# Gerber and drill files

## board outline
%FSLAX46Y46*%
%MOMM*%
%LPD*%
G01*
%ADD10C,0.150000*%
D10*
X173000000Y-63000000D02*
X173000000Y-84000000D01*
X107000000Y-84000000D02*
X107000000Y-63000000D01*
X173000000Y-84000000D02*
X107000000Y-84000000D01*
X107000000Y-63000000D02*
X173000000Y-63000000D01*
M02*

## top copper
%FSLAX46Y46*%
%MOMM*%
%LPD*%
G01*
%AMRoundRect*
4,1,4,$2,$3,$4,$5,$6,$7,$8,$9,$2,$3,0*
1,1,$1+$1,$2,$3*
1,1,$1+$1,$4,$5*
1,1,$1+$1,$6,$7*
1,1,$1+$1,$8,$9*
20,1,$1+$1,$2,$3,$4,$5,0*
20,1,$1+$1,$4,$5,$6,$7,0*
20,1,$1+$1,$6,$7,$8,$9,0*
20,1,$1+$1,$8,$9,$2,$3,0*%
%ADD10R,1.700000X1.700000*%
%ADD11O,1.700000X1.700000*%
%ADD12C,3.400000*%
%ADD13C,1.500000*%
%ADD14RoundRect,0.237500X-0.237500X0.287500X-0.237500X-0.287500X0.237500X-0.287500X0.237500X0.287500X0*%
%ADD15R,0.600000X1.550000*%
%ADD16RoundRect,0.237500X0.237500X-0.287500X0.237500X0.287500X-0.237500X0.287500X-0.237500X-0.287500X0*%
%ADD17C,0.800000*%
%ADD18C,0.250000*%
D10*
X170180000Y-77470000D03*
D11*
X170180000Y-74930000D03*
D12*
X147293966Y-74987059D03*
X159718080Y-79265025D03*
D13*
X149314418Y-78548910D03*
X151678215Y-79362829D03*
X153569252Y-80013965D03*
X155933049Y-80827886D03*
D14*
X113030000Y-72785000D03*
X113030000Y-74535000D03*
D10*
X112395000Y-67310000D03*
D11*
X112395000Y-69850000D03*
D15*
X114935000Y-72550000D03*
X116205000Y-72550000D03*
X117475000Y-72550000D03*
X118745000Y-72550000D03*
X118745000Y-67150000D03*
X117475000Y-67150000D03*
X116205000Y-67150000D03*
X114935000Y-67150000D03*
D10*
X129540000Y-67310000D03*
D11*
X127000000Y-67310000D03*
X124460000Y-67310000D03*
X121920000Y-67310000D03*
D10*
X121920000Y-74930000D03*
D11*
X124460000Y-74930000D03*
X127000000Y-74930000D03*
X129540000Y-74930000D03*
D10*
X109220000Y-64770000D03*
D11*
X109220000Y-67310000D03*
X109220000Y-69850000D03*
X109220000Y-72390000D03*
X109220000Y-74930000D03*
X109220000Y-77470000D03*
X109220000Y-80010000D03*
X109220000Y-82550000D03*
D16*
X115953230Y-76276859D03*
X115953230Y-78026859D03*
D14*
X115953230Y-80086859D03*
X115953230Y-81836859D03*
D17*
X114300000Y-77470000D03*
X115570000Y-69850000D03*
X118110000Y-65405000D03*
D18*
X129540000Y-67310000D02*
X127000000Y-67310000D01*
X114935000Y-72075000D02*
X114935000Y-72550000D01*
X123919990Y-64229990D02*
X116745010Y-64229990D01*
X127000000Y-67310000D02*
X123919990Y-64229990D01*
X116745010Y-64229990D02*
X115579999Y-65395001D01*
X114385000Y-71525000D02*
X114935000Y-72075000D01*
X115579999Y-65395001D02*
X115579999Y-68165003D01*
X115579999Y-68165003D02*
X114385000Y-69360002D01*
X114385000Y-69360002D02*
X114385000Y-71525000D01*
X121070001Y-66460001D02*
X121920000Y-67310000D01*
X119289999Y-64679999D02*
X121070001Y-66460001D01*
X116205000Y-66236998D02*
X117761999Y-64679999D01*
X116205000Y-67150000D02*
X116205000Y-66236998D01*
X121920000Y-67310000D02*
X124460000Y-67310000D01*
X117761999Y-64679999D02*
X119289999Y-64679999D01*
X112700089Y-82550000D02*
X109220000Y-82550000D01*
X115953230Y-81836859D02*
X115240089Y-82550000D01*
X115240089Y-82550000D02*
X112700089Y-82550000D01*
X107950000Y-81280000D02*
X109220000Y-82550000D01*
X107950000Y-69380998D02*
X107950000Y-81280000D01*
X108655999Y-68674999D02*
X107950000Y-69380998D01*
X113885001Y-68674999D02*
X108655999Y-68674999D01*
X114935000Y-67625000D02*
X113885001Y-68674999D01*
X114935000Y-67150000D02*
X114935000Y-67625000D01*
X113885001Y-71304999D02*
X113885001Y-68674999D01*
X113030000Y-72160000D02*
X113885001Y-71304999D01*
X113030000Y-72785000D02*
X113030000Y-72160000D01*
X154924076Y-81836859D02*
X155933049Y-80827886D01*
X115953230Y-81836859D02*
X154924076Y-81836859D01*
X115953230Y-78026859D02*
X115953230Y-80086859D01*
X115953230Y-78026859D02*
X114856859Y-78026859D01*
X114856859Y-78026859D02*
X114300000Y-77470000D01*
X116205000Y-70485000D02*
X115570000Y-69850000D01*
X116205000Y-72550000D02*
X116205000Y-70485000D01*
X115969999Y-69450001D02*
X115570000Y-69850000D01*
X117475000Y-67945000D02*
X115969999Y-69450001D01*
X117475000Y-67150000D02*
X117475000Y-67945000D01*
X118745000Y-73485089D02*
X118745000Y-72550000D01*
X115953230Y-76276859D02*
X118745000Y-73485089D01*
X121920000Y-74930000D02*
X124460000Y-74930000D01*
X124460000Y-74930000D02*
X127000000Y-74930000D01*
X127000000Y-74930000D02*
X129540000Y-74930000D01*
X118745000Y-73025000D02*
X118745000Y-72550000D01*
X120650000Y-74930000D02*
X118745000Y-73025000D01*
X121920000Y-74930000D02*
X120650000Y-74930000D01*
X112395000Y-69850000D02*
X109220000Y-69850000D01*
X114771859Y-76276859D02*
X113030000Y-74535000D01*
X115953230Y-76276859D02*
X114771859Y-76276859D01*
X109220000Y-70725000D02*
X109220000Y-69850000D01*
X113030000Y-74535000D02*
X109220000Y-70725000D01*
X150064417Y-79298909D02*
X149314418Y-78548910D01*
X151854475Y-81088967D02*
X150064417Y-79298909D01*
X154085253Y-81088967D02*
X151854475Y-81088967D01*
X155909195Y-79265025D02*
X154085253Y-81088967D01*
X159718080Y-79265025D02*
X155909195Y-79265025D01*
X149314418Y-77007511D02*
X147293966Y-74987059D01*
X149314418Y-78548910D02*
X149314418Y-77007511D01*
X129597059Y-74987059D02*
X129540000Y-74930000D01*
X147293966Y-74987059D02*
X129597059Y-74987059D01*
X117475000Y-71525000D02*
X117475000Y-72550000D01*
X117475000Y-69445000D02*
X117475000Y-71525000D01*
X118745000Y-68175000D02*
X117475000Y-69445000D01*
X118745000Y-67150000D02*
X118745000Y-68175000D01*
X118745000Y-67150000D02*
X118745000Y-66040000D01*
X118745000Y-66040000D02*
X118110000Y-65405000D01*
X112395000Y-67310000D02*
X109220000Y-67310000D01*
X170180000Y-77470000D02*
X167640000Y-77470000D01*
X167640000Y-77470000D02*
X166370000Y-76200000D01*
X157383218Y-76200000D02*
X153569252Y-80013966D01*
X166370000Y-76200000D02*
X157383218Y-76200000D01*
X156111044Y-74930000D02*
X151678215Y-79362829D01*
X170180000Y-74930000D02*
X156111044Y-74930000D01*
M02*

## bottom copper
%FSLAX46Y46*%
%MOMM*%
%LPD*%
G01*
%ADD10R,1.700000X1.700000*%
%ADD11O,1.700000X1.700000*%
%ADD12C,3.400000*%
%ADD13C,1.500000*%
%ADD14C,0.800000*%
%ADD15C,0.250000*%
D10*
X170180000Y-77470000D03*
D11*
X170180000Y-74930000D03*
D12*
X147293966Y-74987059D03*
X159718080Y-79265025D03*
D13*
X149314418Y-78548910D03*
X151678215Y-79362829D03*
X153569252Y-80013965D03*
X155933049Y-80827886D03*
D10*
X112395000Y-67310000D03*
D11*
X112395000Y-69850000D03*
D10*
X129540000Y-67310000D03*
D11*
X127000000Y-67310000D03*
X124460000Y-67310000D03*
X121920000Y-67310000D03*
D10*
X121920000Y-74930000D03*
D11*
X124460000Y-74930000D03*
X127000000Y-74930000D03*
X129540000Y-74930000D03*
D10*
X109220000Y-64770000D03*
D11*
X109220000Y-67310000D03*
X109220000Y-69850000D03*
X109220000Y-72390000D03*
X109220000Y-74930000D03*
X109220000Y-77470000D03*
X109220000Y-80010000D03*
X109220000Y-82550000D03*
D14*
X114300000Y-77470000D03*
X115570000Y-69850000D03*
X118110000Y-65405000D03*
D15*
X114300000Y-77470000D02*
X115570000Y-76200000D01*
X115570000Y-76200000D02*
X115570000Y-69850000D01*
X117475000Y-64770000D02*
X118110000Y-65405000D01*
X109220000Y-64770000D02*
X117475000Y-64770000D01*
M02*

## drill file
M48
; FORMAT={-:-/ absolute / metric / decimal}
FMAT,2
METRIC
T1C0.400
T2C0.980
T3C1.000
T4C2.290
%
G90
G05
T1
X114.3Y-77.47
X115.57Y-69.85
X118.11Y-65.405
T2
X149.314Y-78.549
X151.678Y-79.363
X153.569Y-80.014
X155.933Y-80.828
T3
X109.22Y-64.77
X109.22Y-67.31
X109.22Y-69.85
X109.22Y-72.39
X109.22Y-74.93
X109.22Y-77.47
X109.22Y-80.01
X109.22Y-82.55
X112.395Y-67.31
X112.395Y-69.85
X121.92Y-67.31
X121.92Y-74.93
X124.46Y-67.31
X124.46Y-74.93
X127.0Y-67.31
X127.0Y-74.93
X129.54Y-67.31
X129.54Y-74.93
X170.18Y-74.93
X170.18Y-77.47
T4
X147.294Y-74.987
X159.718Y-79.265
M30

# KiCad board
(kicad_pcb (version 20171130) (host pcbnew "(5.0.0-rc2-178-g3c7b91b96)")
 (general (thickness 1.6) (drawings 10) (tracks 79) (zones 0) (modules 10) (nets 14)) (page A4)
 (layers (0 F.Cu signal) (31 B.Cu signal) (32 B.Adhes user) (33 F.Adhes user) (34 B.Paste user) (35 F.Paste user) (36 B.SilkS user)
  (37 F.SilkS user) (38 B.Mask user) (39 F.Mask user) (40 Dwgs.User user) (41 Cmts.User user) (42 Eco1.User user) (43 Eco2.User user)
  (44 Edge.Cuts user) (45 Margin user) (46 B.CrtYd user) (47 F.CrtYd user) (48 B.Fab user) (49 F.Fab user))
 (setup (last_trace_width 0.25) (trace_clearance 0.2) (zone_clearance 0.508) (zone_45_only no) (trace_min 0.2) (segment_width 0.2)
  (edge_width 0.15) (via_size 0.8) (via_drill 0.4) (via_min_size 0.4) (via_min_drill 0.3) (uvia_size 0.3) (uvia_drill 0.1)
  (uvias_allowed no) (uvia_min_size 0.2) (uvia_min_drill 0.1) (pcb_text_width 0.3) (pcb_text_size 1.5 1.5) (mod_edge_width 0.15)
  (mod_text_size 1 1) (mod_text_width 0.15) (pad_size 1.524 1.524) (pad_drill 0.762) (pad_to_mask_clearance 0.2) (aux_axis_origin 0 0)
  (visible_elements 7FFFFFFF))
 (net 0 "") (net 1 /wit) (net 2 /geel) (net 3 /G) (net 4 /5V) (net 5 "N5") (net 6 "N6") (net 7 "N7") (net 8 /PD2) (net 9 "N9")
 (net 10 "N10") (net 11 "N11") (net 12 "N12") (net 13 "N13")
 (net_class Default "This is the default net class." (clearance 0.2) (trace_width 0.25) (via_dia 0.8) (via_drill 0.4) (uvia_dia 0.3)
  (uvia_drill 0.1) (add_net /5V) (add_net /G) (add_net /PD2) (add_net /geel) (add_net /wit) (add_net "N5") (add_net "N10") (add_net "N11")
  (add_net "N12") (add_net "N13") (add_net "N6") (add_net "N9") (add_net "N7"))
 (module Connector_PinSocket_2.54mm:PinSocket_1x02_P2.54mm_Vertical (layer B.Cu) (at 170.18 77.47)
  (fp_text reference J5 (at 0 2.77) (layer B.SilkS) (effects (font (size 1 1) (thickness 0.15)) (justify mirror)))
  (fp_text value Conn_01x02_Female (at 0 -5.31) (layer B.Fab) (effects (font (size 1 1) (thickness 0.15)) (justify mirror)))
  (pad 1 thru_hole rect (at 0 0) (size 1.7 1.7) (drill 1) (layers *.Cu *.Mask) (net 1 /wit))
  (pad 2 thru_hole oval (at 0 -2.54) (size 1.7 1.7) (drill 1) (layers *.Cu *.Mask) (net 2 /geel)))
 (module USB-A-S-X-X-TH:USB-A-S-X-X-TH (layer F.Cu) (at 153.506023 77.126042 161)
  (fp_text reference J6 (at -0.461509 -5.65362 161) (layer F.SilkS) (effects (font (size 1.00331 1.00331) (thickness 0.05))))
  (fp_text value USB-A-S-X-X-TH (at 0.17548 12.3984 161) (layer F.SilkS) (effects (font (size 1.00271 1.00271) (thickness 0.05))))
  (pad 6 thru_hole circle (at 6.57 0 161) (size 3.4 3.4) (drill 2.29) (layers *.Cu *.Mask) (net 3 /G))
  (pad 5 thru_hole circle (at -6.57 0 161) (size 3.4 3.4) (drill 2.29) (layers *.Cu *.Mask) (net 3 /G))
  (pad 4 thru_hole circle (at 3.5 -2.710001 161) (size 1.5 1.5) (drill 0.98) (layers *.Cu *.Mask) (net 3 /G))
  (pad 3 thru_hole circle (at 1 -2.71 161) (size 1.5 1.5) (drill 0.98) (layers *.Cu *.Mask) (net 2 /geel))
  (pad 2 thru_hole circle (at -1 -2.71 161) (size 1.5 1.5) (drill 0.98) (layers *.Cu *.Mask) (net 1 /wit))
  (pad 1 thru_hole circle (at -3.500001 -2.71 161) (size 1.5 1.5) (drill 0.98) (layers *.Cu *.Mask) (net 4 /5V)))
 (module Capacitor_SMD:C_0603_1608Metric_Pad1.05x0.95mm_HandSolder (layer F.Cu) (at 113.03 73.66 270)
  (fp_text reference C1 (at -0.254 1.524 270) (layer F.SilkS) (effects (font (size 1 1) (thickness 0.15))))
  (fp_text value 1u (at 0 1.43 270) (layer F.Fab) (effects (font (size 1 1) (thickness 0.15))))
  (pad 1 smd roundrect (at -0.875 0 270) (size 1.05 0.95) (layers F.Cu F.Paste F.Mask) (roundrect_rratio 0.25) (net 4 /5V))
  (pad 2 smd roundrect (at 0.875 0 270) (size 1.05 0.95) (layers F.Cu F.Paste F.Mask) (roundrect_rratio 0.25) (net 3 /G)))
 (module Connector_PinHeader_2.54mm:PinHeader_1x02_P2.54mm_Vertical (layer F.Cu) (at 112.395 67.31)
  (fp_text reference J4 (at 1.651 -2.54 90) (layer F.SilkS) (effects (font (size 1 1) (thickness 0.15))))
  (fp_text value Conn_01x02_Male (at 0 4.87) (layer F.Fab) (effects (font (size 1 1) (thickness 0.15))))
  (pad 1 thru_hole rect (at 0 0) (size 1.7 1.7) (drill 1) (layers *.Cu *.Mask) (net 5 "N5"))
  (pad 2 thru_hole oval (at 0 2.54) (size 1.7 1.7) (drill 1) (layers *.Cu *.Mask) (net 3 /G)))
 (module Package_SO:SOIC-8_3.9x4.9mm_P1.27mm (layer F.Cu) (at 116.84 69.85 90)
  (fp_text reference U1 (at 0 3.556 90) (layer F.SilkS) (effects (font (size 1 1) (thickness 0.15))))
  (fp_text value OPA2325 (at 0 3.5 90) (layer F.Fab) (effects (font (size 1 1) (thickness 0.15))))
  (pad 1 smd rect (at -2.7 -1.905 90) (size 1.55 0.6) (layers F.Cu F.Paste F.Mask) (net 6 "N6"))
  (pad 2 smd rect (at -2.7 -0.635 90) (size 1.55 0.6) (layers F.Cu F.Paste F.Mask) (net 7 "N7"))
  (pad 3 smd rect (at -2.7 0.635 90) (size 1.55 0.6) (layers F.Cu F.Paste F.Mask) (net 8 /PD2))
  (pad 4 smd rect (at -2.7 1.905 90) (size 1.55 0.6) (layers F.Cu F.Paste F.Mask) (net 3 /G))
  (pad 5 smd rect (at 2.7 1.905 90) (size 1.55 0.6) (layers F.Cu F.Paste F.Mask) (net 8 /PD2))
  (pad 6 smd rect (at 2.7 0.635 90) (size 1.55 0.6) (layers F.Cu F.Paste F.Mask) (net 7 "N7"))
  (pad 7 smd rect (at 2.7 -0.635 90) (size 1.55 0.6) (layers F.Cu F.Paste F.Mask) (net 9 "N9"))
  (pad 8 smd rect (at 2.7 -1.905 90) (size 1.55 0.6) (layers F.Cu F.Paste F.Mask) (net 4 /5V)))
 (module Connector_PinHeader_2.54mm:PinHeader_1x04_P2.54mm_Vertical (layer F.Cu) (at 129.54 67.31 270)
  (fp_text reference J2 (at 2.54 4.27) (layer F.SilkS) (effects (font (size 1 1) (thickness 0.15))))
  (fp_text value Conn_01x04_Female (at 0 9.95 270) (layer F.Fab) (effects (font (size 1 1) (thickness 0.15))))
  (pad 1 thru_hole rect (at 0 0 270) (size 1.7 1.7) (drill 1) (layers *.Cu *.Mask) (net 6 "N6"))
  (pad 2 thru_hole oval (at 0 2.54 270) (size 1.7 1.7) (drill 1) (layers *.Cu *.Mask) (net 6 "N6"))
  (pad 3 thru_hole oval (at 0 5.08 270) (size 1.7 1.7) (drill 1) (layers *.Cu *.Mask) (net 9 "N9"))
  (pad 4 thru_hole oval (at 0 7.62 270) (size 1.7 1.7) (drill 1) (layers *.Cu *.Mask) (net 9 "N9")))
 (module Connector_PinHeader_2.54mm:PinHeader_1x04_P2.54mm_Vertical (layer F.Cu) (at 121.92 74.93 90)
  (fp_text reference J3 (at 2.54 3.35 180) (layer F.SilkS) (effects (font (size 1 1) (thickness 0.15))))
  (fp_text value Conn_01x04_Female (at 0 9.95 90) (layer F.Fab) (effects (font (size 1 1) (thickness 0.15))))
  (pad 1 thru_hole rect (at 0 0 90) (size 1.7 1.7) (drill 1) (layers *.Cu *.Mask) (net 3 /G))
  (pad 2 thru_hole oval (at 0 2.54 90) (size 1.7 1.7) (drill 1) (layers *.Cu *.Mask) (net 3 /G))
  (pad 3 thru_hole oval (at 0 5.08 90) (size 1.7 1.7) (drill 1) (layers *.Cu *.Mask) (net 3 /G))
  (pad 4 thru_hole oval (at 0 7.62 90) (size 1.7 1.7) (drill 1) (layers *.Cu *.Mask) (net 3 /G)))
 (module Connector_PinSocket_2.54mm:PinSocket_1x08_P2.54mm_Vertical (layer B.Cu) (at 109.22 64.77 180)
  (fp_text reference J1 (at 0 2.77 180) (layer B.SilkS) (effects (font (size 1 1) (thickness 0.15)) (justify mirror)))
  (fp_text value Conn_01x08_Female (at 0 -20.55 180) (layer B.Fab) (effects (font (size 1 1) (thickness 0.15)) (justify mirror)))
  (pad 1 thru_hole rect (at 0 0 180) (size 1.7 1.7) (drill 1) (layers *.Cu *.Mask) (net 8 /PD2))
  (pad 2 thru_hole oval (at 0 -2.54 180) (size 1.7 1.7) (drill 1) (layers *.Cu *.Mask) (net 5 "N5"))
  (pad 3 thru_hole oval (at 0 -5.08 180) (size 1.7 1.7) (drill 1) (layers *.Cu *.Mask) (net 3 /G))
  (pad 4 thru_hole oval (at 0 -7.62 180) (size 1.7 1.7) (drill 1) (layers *.Cu *.Mask) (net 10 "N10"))
  (pad 5 thru_hole oval (at 0 -10.16 180) (size 1.7 1.7) (drill 1) (layers *.Cu *.Mask) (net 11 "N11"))
  (pad 6 thru_hole oval (at 0 -12.7 180) (size 1.7 1.7) (drill 1) (layers *.Cu *.Mask) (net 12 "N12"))
  (pad 7 thru_hole oval (at 0 -15.24 180) (size 1.7 1.7) (drill 1) (layers *.Cu *.Mask) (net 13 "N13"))
  (pad 8 thru_hole oval (at 0 -17.78 180) (size 1.7 1.7) (drill 1) (layers *.Cu *.Mask) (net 4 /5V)))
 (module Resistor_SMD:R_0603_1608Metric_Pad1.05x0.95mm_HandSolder (layer F.Cu) (at 115.95323 77.151859 90)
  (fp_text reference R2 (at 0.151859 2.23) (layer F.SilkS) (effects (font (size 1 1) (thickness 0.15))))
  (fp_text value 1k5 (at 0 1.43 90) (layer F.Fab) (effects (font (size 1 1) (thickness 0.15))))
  (pad 2 smd roundrect (at 0.875 0 90) (size 1.05 0.95) (layers F.Cu F.Paste F.Mask) (roundrect_rratio 0.25) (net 3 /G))
  (pad 1 smd roundrect (at -0.875 0 90) (size 1.05 0.95) (layers F.Cu F.Paste F.Mask) (roundrect_rratio 0.25) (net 7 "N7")))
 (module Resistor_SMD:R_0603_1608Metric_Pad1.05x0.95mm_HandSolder (layer F.Cu) (at 115.95323 80.961859 270)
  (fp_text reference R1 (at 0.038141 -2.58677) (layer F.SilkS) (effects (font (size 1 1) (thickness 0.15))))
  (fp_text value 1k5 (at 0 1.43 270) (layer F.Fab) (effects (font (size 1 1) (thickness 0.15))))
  (pad 1 smd roundrect (at -0.875 0 270) (size 1.05 0.95) (layers F.Cu F.Paste F.Mask) (roundrect_rratio 0.25) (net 7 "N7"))
  (pad 2 smd roundrect (at 0.875 0 270) (size 1.05 0.95) (layers F.Cu F.Paste F.Mask) (roundrect_rratio 0.25) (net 4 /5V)))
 (gr_line (start 173 63) (end 173 84) (layer Edge.Cuts) (width 0.15))
 (gr_line (start 107 84) (end 107 63) (layer Edge.Cuts) (width 0.15))
 (gr_line (start 173 84) (end 107 84) (layer Edge.Cuts) (width 0.15))
 (gr_line (start 107 63) (end 173 63) (layer Edge.Cuts) (width 0.15))
 (segment (start 129.54 67.31) (end 127 67.31) (width 0.25) (layer F.Cu) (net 6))
 (segment (start 114.935 72.075) (end 114.935 72.55) (width 0.25) (layer F.Cu) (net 6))
 (segment (start 123.91999 64.22999) (end 116.74501 64.22999) (width 0.25) (layer F.Cu) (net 6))
 (segment (start 127 67.31) (end 123.91999 64.22999) (width 0.25) (layer F.Cu) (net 6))
 (segment (start 116.74501 64.22999) (end 115.579999 65.395001) (width 0.25) (layer F.Cu) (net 6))
 (segment (start 114.385 71.525) (end 114.935 72.075) (width 0.25) (layer F.Cu) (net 6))
 (segment (start 115.579999 65.395001) (end 115.579999 68.165003) (width 0.25) (layer F.Cu) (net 6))
 (segment (start 115.579999 68.165003) (end 114.385 69.360002) (width 0.25) (layer F.Cu) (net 6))
 (segment (start 114.385 69.360002) (end 114.385 71.525) (width 0.25) (layer F.Cu) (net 6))
 (segment (start 121.070001 66.460001) (end 121.92 67.31) (width 0.25) (layer F.Cu) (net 9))
 (segment (start 119.289999 64.679999) (end 121.070001 66.460001) (width 0.25) (layer F.Cu) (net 9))
 (segment (start 116.205 66.236998) (end 117.761999 64.679999) (width 0.25) (layer F.Cu) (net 9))
 (segment (start 116.205 67.15) (end 116.205 66.236998) (width 0.25) (layer F.Cu) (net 9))
 (segment (start 121.92 67.31) (end 124.46 67.31) (width 0.25) (layer F.Cu) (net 9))
 (segment (start 117.761999 64.679999) (end 119.289999 64.679999) (width 0.25) (layer F.Cu) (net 9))
 (segment (start 112.700089 82.55) (end 109.22 82.55) (width 0.25) (layer F.Cu) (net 4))
 (segment (start 115.95323 81.836859) (end 115.240089 82.55) (width 0.25) (layer F.Cu) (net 4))
 (segment (start 115.240089 82.55) (end 112.700089 82.55) (width 0.25) (layer F.Cu) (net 4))
 (segment (start 107.95 81.28) (end 109.22 82.55) (width 0.25) (layer F.Cu) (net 4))
 (segment (start 107.95 69.380998) (end 107.95 81.28) (width 0.25) (layer F.Cu) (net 4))
 (segment (start 108.655999 68.674999) (end 107.95 69.380998) (width 0.25) (layer F.Cu) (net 4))
 (segment (start 113.885001 68.674999) (end 108.655999 68.674999) (width 0.25) (layer F.Cu) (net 4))
 (segment (start 114.935 67.625) (end 113.885001 68.674999) (width 0.25) (layer F.Cu) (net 4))
 (segment (start 114.935 67.15) (end 114.935 67.625) (width 0.25) (layer F.Cu) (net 4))
 (segment (start 113.885001 71.304999) (end 113.885001 68.674999) (width 0.25) (layer F.Cu) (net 4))
 (segment (start 113.03 72.16) (end 113.885001 71.304999) (width 0.25) (layer F.Cu) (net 4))
 (segment (start 113.03 72.785) (end 113.03 72.16) (width 0.25) (layer F.Cu) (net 4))
 (segment (start 154.924076 81.836859) (end 155.933049 80.827886) (width 0.25) (layer F.Cu) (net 4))
 (segment (start 115.95323 81.836859) (end 154.924076 81.836859) (width 0.25) (layer F.Cu) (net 4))
 (segment (start 115.95323 78.026859) (end 115.95323 80.086859) (width 0.25) (layer F.Cu) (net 7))
 (via (at 114.3 77.47) (size 0.8) (drill 0.4) (layers F.Cu B.Cu) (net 7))
 (segment (start 115.95323 78.026859) (end 114.856859 78.026859) (width 0.25) (layer F.Cu) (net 7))
 (segment (start 114.856859 78.026859) (end 114.3 77.47) (width 0.25) (layer F.Cu) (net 7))
 (via (at 115.57 69.85) (size 0.8) (drill 0.4) (layers F.Cu B.Cu) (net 7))
 (segment (start 114.3 77.47) (end 115.57 76.2) (width 0.25) (layer B.Cu) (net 7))
 (segment (start 115.57 76.2) (end 115.57 69.85) (width 0.25) (layer B.Cu) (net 7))
 (segment (start 116.205 70.485) (end 115.57 69.85) (width 0.25) (layer F.Cu) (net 7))
 (segment (start 116.205 72.55) (end 116.205 70.485) (width 0.25) (layer F.Cu) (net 7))
 (segment (start 115.969999 69.450001) (end 115.57 69.85) (width 0.25) (layer F.Cu) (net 7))
 (segment (start 117.475 67.945) (end 115.969999 69.450001) (width 0.25) (layer F.Cu) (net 7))
 (segment (start 117.475 67.15) (end 117.475 67.945) (width 0.25) (layer F.Cu) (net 7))
 (segment (start 118.745 73.485089) (end 118.745 72.55) (width 0.25) (layer F.Cu) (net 3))
 (segment (start 115.95323 76.276859) (end 118.745 73.485089) (width 0.25) (layer F.Cu) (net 3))
 (segment (start 121.92 74.93) (end 124.46 74.93) (width 0.25) (layer F.Cu) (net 3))
 (segment (start 124.46 74.93) (end 127 74.93) (width 0.25) (layer F.Cu) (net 3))
 (segment (start 127 74.93) (end 129.54 74.93) (width 0.25) (layer F.Cu) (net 3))
 (segment (start 118.745 73.025) (end 118.745 72.55) (width 0.25) (layer F.Cu) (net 3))
 (segment (start 120.65 74.93) (end 118.745 73.025) (width 0.25) (layer F.Cu) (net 3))
 (segment (start 121.92 74.93) (end 120.65 74.93) (width 0.25) (layer F.Cu) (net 3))
 (segment (start 112.395 69.85) (end 109.22 69.85) (width 0.25) (layer F.Cu) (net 3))
 (segment (start 114.771859 76.276859) (end 113.03 74.535) (width 0.25) (layer F.Cu) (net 3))
 (segment (start 115.95323 76.276859) (end 114.771859 76.276859) (width 0.25) (layer F.Cu) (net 3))
 (segment (start 109.22 70.725) (end 109.22 69.85) (width 0.25) (layer F.Cu) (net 3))
 (segment (start 113.03 74.535) (end 109.22 70.725) (width 0.25) (layer F.Cu) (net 3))
 (segment (start 150.064417 79.298909) (end 149.314418 78.54891) (width 0.25) (layer F.Cu) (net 3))
 (segment (start 151.854475 81.088967) (end 150.064417 79.298909) (width 0.25) (layer F.Cu) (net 3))
 (segment (start 154.085253 81.088967) (end 151.854475 81.088967) (width 0.25) (layer F.Cu) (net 3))
 (segment (start 155.909195 79.265025) (end 154.085253 81.088967) (width 0.25) (layer F.Cu) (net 3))
 (segment (start 159.71808 79.265025) (end 155.909195 79.265025) (width 0.25) (layer F.Cu) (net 3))
 (segment (start 149.314418 77.007511) (end 147.293966 74.987059) (width 0.25) (layer F.Cu) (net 3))
 (segment (start 149.314418 78.54891) (end 149.314418 77.007511) (width 0.25) (layer F.Cu) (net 3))
 (segment (start 129.597059 74.987059) (end 129.54 74.93) (width 0.25) (layer F.Cu) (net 3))
 (segment (start 147.293966 74.987059) (end 129.597059 74.987059) (width 0.25) (layer F.Cu) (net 3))
 (segment (start 117.475 71.525) (end 117.475 72.55) (width 0.25) (layer F.Cu) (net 8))
 (segment (start 117.475 69.445) (end 117.475 71.525) (width 0.25) (layer F.Cu) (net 8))
 (segment (start 118.745 68.175) (end 117.475 69.445) (width 0.25) (layer F.Cu) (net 8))
 (segment (start 118.745 67.15) (end 118.745 68.175) (width 0.25) (layer F.Cu) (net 8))
 (via (at 118.11 65.405) (size 0.8) (drill 0.4) (layers F.Cu B.Cu) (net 8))
 (segment (start 118.745 67.15) (end 118.745 66.04) (width 0.25) (layer F.Cu) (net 8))
 (segment (start 118.745 66.04) (end 118.11 65.405) (width 0.25) (layer F.Cu) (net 8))
 (segment (start 117.475 64.77) (end 118.11 65.405) (width 0.25) (layer B.Cu) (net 8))
 (segment (start 109.22 64.77) (end 117.475 64.77) (width 0.25) (layer B.Cu) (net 8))
 (segment (start 112.395 67.31) (end 109.22 67.31) (width 0.25) (layer F.Cu) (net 5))
 (segment (start 170.18 77.47) (end 167.64 77.47) (width 0.25) (layer F.Cu) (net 1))
 (segment (start 167.64 77.47) (end 166.37 76.2) (width 0.25) (layer F.Cu) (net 1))
 (segment (start 157.383218 76.2) (end 153.569252 80.013966) (width 0.25) (layer F.Cu) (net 1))
 (segment (start 166.37 76.2) (end 157.383218 76.2) (width 0.25) (layer F.Cu) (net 1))
 (segment (start 156.111044 74.93) (end 151.678215 79.362829) (width 0.25) (layer F.Cu) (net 2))
 (segment (start 170.18 74.93) (end 156.111044 74.93) (width 0.25) (layer F.Cu) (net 2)))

